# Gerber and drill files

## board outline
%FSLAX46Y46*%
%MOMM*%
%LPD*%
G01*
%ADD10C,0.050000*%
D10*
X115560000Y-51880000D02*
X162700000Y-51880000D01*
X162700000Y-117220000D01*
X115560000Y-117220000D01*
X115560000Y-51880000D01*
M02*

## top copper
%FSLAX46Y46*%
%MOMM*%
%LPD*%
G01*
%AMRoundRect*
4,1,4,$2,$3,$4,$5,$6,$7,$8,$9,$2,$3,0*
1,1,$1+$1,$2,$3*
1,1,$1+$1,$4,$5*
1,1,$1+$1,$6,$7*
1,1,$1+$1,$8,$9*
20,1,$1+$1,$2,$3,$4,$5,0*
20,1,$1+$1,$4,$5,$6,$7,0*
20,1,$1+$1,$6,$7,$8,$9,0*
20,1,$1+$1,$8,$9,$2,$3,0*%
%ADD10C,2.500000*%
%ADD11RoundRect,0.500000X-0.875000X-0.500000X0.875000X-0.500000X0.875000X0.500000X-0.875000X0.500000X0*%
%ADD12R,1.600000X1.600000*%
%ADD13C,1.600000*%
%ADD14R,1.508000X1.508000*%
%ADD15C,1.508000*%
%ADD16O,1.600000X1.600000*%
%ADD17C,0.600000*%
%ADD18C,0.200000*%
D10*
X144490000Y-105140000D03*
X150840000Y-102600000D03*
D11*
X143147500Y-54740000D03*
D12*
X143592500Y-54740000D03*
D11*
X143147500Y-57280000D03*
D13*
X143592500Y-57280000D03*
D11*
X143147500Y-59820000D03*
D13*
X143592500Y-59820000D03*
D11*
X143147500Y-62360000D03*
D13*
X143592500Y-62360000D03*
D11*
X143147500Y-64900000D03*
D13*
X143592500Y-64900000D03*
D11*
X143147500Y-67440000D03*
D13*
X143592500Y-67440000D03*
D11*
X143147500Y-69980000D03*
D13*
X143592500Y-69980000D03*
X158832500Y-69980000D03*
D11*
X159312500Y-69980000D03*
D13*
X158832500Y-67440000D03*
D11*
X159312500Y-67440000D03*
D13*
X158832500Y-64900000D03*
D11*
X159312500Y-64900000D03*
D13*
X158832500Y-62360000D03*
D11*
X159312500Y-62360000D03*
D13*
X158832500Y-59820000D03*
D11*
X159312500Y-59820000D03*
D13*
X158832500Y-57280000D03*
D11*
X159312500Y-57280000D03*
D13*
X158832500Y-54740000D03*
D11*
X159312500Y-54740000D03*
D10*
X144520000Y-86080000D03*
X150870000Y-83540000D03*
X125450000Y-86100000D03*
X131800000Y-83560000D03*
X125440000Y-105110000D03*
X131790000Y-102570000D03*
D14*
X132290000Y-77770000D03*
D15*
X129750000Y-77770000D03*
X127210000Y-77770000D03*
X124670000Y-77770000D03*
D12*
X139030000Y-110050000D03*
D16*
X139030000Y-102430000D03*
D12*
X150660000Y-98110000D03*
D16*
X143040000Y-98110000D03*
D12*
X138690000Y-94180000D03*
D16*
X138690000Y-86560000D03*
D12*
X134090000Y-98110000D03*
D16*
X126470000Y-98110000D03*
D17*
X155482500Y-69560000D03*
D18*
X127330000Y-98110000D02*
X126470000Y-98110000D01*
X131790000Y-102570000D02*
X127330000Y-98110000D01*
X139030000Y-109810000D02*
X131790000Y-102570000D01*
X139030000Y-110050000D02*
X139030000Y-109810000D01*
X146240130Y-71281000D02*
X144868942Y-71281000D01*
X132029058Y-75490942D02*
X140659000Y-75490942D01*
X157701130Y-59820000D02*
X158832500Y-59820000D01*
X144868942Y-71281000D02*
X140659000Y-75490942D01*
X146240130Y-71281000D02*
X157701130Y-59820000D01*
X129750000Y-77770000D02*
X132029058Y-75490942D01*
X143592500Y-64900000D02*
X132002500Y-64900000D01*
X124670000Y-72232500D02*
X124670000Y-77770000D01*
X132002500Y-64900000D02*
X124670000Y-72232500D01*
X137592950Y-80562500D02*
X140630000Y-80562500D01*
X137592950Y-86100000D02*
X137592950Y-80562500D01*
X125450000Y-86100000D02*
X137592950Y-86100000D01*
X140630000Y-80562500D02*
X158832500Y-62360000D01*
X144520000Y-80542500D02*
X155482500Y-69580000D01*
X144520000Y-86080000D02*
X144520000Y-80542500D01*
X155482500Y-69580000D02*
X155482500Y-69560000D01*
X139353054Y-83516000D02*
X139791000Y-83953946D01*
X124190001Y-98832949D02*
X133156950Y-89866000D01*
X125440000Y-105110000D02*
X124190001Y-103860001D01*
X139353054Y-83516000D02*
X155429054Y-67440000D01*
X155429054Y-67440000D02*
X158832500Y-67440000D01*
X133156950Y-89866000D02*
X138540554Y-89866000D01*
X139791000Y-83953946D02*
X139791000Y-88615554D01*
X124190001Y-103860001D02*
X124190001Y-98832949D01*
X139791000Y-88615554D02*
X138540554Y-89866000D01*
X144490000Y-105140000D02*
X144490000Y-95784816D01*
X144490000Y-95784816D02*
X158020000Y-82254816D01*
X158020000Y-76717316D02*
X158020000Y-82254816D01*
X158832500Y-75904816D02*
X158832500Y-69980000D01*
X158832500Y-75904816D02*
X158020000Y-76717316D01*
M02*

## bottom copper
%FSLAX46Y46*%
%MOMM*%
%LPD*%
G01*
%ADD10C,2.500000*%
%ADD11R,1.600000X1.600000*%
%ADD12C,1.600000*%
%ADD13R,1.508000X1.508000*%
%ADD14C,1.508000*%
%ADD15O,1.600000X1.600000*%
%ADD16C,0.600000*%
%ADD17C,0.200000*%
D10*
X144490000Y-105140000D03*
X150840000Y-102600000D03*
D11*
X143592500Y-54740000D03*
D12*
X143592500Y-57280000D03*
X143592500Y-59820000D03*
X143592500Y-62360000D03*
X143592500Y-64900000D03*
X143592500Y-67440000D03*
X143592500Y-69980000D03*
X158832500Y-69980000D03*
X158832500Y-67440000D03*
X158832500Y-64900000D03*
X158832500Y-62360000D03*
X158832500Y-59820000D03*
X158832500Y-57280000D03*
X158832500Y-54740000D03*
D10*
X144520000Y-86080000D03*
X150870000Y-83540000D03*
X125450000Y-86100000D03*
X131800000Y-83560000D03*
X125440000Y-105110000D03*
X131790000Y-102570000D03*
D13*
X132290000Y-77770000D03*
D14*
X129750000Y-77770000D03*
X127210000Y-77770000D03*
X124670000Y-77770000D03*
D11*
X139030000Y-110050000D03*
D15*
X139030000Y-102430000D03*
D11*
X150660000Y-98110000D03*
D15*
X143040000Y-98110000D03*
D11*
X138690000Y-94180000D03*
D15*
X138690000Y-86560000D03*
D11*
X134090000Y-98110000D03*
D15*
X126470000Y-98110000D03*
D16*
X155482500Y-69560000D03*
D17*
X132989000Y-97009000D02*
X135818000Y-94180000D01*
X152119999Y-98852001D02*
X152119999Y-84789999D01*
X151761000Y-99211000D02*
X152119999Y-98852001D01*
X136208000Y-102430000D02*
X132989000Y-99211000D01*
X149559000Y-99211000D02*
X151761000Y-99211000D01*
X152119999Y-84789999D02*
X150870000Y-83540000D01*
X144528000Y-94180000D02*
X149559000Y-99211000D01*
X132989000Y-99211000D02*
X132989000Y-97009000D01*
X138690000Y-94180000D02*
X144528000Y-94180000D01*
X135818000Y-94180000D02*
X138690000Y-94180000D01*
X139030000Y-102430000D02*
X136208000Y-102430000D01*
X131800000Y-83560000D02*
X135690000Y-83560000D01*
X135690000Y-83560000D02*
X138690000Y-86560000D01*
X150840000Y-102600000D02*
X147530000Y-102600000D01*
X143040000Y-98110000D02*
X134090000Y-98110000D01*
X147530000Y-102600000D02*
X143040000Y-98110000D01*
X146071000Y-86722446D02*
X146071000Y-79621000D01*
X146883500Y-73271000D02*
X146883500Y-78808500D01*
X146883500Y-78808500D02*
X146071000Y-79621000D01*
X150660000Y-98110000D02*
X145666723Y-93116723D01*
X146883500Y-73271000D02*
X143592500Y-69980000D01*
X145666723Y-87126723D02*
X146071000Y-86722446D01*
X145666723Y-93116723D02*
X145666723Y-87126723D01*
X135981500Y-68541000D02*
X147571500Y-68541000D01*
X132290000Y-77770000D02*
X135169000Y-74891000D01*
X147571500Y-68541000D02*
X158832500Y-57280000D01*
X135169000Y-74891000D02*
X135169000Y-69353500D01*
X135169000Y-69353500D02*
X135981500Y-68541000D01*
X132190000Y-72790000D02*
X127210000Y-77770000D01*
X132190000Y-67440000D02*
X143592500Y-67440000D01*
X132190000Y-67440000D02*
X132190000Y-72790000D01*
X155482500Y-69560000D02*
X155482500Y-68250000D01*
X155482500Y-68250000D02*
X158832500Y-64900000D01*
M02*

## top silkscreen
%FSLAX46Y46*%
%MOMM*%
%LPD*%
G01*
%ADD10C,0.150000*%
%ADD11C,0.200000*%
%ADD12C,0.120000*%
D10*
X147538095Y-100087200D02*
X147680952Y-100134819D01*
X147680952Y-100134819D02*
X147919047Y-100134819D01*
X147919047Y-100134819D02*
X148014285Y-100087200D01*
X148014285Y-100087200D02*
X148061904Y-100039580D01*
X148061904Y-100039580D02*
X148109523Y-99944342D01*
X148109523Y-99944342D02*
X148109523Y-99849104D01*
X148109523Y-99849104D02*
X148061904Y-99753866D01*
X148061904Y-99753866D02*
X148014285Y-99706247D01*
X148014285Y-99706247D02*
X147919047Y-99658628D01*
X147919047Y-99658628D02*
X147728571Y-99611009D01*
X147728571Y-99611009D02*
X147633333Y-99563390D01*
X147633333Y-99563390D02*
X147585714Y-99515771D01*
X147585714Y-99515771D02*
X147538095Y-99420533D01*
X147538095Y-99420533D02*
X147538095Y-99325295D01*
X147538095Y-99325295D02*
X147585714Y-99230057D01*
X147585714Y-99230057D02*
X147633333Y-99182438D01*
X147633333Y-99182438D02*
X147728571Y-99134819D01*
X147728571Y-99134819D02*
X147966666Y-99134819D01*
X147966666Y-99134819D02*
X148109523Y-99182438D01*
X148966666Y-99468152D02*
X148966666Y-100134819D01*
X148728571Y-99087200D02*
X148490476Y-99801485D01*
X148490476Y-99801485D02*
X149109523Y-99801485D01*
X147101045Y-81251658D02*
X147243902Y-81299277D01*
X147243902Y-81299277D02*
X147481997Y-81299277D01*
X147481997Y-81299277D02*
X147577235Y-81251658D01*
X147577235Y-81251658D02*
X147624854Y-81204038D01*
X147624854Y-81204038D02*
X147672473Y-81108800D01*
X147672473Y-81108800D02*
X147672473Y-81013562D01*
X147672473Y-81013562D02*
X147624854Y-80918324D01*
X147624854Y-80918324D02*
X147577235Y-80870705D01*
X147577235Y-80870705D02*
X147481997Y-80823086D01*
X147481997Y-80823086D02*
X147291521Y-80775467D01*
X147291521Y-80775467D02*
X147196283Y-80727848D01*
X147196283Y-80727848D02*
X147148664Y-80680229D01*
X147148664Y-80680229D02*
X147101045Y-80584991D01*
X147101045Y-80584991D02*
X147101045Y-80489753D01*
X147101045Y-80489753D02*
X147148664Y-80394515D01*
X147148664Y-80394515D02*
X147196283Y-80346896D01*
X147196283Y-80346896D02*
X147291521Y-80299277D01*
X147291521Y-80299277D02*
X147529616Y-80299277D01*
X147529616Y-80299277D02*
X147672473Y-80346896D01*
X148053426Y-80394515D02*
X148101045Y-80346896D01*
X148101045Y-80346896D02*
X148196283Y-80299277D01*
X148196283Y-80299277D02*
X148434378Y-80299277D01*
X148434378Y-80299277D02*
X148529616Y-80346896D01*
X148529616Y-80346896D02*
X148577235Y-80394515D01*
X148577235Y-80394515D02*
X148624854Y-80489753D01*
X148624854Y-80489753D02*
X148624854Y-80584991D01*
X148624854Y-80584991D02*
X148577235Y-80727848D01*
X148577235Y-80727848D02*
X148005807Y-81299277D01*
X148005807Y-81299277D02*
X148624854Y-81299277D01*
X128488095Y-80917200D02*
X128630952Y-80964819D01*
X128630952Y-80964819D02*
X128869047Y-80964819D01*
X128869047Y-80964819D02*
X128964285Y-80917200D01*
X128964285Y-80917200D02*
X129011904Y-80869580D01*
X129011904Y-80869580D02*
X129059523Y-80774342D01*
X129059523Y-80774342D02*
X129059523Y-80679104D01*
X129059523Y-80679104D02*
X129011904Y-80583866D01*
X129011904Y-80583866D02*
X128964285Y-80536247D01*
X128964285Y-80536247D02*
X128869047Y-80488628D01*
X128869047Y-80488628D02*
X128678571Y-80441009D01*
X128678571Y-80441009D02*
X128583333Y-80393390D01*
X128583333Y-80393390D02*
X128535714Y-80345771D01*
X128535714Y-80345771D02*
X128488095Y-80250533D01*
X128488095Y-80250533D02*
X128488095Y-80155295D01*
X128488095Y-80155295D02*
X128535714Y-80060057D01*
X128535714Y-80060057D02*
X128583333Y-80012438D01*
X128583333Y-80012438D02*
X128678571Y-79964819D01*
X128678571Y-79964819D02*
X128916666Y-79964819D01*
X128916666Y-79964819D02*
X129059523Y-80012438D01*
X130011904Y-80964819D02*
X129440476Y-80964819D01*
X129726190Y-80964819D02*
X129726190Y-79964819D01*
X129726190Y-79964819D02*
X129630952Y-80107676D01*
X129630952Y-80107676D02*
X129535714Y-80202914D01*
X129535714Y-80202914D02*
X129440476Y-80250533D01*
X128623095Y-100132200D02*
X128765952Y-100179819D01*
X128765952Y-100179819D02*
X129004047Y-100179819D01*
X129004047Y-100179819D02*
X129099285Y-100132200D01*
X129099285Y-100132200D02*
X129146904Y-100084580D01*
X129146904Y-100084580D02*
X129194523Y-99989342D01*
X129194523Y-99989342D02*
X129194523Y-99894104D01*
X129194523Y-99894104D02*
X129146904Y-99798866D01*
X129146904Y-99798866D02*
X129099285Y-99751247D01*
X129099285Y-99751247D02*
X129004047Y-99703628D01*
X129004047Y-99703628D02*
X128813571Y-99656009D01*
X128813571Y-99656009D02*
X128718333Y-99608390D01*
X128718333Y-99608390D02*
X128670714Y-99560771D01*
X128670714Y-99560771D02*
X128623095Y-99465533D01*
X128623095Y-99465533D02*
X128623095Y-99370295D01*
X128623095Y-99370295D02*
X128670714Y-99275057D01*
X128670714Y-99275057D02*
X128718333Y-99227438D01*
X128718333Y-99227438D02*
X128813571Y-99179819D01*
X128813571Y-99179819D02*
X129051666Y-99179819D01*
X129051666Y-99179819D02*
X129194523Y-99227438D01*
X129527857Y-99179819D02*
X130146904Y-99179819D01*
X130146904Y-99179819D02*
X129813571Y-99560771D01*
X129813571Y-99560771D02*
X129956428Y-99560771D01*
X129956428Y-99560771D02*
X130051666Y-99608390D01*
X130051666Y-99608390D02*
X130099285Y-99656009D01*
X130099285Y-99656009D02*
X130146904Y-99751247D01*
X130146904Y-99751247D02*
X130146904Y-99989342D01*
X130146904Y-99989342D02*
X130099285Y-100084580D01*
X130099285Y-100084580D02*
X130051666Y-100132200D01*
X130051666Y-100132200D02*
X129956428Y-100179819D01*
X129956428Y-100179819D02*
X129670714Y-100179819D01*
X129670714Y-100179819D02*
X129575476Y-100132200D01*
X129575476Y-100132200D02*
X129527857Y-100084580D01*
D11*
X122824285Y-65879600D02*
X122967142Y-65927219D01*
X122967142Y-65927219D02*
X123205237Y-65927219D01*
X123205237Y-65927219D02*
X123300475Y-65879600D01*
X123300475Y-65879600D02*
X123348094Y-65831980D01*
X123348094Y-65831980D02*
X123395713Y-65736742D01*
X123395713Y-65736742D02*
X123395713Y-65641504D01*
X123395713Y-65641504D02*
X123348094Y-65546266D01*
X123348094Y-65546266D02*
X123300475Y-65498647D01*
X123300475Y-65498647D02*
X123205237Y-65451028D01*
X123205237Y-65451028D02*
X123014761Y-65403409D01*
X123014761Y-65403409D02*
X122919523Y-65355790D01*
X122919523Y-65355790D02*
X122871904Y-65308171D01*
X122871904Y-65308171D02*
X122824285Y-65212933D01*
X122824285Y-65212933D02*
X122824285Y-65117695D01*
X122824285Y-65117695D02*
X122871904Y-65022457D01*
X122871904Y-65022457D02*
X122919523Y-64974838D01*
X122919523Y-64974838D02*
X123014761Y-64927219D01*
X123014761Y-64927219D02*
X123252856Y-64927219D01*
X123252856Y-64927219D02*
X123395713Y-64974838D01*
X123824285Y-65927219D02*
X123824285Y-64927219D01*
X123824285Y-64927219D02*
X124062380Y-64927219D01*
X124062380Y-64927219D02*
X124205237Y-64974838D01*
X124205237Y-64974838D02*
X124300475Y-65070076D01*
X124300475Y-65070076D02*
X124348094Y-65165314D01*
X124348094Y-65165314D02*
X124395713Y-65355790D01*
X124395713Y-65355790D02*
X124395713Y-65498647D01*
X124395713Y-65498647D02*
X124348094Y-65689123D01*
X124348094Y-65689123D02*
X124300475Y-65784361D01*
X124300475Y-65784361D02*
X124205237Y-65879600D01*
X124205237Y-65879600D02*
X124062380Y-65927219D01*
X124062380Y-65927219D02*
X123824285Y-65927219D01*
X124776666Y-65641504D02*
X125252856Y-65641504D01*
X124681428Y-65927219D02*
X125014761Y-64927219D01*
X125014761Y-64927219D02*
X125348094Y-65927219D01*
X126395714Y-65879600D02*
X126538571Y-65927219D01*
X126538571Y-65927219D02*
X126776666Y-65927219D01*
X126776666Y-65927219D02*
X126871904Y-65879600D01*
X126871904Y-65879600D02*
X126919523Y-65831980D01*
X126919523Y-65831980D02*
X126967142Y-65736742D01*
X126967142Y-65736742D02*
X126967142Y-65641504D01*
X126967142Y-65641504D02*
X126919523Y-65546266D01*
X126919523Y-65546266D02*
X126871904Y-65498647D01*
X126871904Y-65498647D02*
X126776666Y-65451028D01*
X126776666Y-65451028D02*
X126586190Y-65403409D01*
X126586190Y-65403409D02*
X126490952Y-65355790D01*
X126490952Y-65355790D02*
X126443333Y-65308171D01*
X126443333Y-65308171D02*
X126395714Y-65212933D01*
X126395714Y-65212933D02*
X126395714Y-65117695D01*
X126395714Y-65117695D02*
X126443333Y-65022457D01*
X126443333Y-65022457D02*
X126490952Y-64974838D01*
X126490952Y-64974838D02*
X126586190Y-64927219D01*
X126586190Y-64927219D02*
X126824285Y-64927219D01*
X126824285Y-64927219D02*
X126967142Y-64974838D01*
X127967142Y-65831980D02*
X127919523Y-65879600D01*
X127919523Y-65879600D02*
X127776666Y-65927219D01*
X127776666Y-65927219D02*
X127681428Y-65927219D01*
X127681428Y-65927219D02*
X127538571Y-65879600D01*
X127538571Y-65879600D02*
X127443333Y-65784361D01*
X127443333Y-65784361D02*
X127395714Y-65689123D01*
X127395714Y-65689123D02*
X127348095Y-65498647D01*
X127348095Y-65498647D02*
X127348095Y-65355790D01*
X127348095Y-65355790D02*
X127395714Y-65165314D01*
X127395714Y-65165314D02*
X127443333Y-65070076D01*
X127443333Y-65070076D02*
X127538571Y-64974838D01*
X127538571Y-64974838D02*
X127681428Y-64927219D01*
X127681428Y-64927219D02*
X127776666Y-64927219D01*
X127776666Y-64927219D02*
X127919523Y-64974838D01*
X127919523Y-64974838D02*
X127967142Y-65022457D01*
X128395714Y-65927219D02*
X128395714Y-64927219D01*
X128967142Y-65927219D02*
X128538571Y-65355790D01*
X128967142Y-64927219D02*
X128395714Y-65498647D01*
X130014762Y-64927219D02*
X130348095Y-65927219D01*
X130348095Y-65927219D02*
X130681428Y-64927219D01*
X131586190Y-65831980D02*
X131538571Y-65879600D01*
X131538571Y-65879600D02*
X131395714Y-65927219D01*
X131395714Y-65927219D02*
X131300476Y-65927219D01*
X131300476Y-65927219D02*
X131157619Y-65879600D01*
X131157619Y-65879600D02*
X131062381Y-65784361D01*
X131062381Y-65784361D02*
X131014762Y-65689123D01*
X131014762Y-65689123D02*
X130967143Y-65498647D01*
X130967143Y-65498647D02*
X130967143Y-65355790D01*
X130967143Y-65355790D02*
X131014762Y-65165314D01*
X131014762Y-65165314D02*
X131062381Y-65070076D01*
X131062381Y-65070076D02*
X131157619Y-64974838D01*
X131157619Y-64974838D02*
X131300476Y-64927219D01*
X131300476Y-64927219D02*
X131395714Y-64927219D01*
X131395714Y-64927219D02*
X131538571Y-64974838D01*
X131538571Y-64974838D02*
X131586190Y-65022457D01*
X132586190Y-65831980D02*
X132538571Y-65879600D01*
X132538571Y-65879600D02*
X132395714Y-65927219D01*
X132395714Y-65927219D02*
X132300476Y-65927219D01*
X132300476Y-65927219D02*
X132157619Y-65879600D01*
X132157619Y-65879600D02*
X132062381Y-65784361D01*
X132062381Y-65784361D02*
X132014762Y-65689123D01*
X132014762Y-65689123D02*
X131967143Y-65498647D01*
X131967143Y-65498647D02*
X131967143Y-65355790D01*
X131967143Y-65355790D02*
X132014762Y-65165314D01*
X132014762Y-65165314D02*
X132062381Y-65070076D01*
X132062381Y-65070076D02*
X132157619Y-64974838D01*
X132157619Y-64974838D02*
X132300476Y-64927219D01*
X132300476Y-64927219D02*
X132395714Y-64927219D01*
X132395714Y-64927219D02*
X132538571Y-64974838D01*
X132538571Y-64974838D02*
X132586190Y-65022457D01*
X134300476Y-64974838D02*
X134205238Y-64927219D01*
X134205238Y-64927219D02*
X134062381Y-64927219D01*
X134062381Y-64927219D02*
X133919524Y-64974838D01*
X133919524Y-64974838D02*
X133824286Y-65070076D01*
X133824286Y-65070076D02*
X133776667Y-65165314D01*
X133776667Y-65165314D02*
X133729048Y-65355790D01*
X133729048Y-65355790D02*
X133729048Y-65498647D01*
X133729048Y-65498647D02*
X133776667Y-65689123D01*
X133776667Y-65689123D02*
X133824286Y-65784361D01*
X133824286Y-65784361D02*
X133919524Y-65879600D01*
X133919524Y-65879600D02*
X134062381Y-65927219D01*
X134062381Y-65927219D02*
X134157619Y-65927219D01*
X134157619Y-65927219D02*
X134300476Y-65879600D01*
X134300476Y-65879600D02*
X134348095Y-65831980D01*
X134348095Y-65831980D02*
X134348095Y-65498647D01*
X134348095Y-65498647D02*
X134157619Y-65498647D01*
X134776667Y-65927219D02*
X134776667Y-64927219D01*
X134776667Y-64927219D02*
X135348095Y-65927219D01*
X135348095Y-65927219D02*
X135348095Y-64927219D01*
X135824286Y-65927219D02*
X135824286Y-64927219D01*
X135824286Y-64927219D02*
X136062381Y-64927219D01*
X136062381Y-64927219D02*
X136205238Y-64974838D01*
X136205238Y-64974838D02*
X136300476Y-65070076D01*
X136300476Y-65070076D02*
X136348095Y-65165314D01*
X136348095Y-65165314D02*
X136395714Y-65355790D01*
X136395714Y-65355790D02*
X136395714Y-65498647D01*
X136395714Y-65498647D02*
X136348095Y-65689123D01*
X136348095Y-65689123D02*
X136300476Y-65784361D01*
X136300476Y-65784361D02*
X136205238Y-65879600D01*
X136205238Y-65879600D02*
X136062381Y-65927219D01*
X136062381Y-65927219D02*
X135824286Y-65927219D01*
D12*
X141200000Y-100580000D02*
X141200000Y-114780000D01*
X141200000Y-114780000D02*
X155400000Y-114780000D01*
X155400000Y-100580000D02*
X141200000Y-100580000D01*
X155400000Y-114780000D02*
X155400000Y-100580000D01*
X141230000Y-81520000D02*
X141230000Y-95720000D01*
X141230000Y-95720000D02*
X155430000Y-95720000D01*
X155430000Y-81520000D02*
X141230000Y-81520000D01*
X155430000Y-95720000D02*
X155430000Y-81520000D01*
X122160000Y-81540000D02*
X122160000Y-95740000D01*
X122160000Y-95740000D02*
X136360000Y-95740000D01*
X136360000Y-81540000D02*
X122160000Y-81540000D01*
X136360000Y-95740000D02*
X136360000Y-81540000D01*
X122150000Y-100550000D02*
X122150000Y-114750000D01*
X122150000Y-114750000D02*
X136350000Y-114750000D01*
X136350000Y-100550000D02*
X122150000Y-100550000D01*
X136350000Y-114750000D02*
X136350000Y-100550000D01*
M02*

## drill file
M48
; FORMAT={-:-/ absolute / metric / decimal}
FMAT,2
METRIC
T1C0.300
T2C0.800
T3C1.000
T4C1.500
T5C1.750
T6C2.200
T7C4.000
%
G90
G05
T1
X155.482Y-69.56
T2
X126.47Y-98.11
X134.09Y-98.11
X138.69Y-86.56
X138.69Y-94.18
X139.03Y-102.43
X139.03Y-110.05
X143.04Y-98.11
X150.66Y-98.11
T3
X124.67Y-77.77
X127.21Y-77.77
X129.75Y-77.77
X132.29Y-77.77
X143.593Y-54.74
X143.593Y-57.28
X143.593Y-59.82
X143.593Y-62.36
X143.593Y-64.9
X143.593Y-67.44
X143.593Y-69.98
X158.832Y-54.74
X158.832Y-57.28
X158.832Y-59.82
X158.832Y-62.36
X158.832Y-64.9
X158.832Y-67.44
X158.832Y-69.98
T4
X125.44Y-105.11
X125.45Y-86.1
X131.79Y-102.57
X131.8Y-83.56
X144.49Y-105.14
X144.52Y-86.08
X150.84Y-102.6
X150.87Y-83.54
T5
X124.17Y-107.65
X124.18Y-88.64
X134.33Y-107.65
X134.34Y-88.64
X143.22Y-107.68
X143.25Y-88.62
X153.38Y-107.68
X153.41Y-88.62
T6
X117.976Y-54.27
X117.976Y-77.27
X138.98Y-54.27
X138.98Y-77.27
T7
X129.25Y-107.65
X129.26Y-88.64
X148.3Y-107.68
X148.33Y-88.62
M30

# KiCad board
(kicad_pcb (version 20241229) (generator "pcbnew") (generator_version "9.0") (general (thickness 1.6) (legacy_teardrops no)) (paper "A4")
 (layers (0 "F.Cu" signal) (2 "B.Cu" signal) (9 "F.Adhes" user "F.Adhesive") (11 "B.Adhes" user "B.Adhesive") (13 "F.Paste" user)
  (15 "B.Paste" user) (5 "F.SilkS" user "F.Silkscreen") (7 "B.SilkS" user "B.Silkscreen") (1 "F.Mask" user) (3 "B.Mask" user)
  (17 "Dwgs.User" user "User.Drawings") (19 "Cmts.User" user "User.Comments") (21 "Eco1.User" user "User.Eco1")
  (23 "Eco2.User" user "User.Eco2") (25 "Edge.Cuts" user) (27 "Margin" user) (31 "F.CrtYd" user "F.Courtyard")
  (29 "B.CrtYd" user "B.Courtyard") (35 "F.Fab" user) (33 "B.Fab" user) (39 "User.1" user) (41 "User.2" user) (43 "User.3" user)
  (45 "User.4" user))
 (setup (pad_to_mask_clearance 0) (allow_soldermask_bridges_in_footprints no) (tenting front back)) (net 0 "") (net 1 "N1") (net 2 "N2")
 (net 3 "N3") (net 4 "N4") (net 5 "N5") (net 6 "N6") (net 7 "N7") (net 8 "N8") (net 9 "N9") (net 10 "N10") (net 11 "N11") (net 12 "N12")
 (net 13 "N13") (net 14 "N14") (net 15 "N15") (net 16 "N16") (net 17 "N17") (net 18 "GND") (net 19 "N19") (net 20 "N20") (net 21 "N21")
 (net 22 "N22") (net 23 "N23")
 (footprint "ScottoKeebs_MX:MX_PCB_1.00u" (layer "F.Cu") (at 148.3 107.68)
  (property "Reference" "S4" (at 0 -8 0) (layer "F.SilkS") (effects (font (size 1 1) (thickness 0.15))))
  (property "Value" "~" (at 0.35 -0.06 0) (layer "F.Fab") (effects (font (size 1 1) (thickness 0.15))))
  (fp_line (start -7.1 -7.1) (end -7.1 7.1) (stroke (width 0.12) (type solid)) (layer "F.SilkS"))
  (fp_line (start -7.1 7.1) (end 7.1 7.1) (stroke (width 0.12) (type solid)) (layer "F.SilkS"))
  (fp_line (start 7.1 -7.1) (end -7.1 -7.1) (stroke (width 0.12) (type solid)) (layer "F.SilkS"))
  (fp_line (start 7.1 7.1) (end 7.1 -7.1) (stroke (width 0.12) (type solid)) (layer "F.SilkS"))
  (pad "" np_thru_hole circle (at -5.08 0) (size 1.75 1.75) (drill 1.75) (layers "*.Cu" "*.Mask"))
  (pad "" np_thru_hole circle (at 0 0) (size 4 4) (drill 4) (layers "*.Cu" "*.Mask"))
  (pad "" np_thru_hole circle (at 5.08 0) (size 1.75 1.75) (drill 1.75) (layers "*.Cu" "*.Mask"))
  (pad "1" thru_hole circle (at -3.81 -2.54) (size 2.5 2.5) (drill 1.5) (layers "*.Cu" "*.Mask") (remove_unused_layers no) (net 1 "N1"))
  (pad "2" thru_hole circle (at 2.54 -5.08) (size 2.5 2.5) (drill 1.5) (layers "*.Cu" "*.Mask") (remove_unused_layers no) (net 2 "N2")))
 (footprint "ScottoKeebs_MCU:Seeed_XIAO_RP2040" (layer "F.Cu") (at 151.2125 62.36)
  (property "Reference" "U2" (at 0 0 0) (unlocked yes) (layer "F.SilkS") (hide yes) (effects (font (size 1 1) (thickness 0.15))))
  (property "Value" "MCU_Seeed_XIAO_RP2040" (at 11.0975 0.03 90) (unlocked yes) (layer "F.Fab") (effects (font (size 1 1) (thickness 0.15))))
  (pad "1" smd roundrect (at -8.065 -7.62) (size 2.75 2) (layers "F.Cu" "F.Mask" "F.Paste") (roundrect_rratio 0.25) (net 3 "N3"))
  (pad "1" thru_hole rect (at -7.62 -7.62 90) (size 1.6 1.6) (drill 1) (layers "*.Cu" "*.Mask") (remove_unused_layers no) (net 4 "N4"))
  (pad "2" smd roundrect (at -8.065 -5.08) (size 2.75 2) (layers "F.Cu" "F.Mask" "F.Paste") (roundrect_rratio 0.25) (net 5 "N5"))
  (pad "2" thru_hole circle (at -7.62 -5.08 90) (size 1.6 1.6) (drill 1) (layers "*.Cu" "*.Mask") (remove_unused_layers no) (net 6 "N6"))
  (pad "3" smd roundrect (at -8.065 -2.54) (size 2.75 2) (layers "F.Cu" "F.Mask" "F.Paste") (roundrect_rratio 0.25) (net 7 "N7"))
  (pad "3" thru_hole circle (at -7.62 -2.54 90) (size 1.6 1.6) (drill 1) (layers "*.Cu" "*.Mask") (remove_unused_layers no) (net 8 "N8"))
  (pad "4" smd roundrect (at -8.065 0) (size 2.75 2) (layers "F.Cu" "F.Mask" "F.Paste") (roundrect_rratio 0.25) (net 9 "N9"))
  (pad "4" thru_hole circle (at -7.62 0 90) (size 1.6 1.6) (drill 1) (layers "*.Cu" "*.Mask") (remove_unused_layers no) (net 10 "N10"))
  (pad "5" smd roundrect (at -8.065 2.54) (size 2.75 2) (layers "F.Cu" "F.Mask" "F.Paste") (roundrect_rratio 0.25) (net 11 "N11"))
  (pad "5" thru_hole circle (at -7.62 2.54 90) (size 1.6 1.6) (drill 1) (layers "*.Cu" "*.Mask") (remove_unused_layers no) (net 11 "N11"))
  (pad "6" smd roundrect (at -8.065 5.08) (size 2.75 2) (layers "F.Cu" "F.Mask" "F.Paste") (roundrect_rratio 0.25) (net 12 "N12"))
  (pad "6" thru_hole circle (at -7.62 5.08 90) (size 1.6 1.6) (drill 1) (layers "*.Cu" "*.Mask") (remove_unused_layers no) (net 12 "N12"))
  (pad "7" smd roundrect (at -8.065 7.62) (size 2.75 2) (layers "F.Cu" "F.Mask" "F.Paste") (roundrect_rratio 0.25) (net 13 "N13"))
  (pad "7" thru_hole circle (at -7.62 7.62 90) (size 1.6 1.6) (drill 1) (layers "*.Cu" "*.Mask") (remove_unused_layers no) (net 13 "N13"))
  (pad "8" thru_hole circle (at 7.62 7.62 90) (size 1.6 1.6) (drill 1) (layers "*.Cu" "*.Mask") (remove_unused_layers no) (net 1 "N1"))
  (pad "8" smd roundrect (at 8.1 7.62) (size 2.75 2) (layers "F.Cu" "F.Mask" "F.Paste") (roundrect_rratio 0.25) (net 1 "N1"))
  (pad "9" thru_hole circle (at 7.62 5.08 90) (size 1.6 1.6) (drill 1) (layers "*.Cu" "*.Mask") (remove_unused_layers no) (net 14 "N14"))
  (pad "9" smd roundrect (at 8.1 5.08) (size 2.75 2) (layers "F.Cu" "F.Mask" "F.Paste") (roundrect_rratio 0.25) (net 14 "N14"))
  (pad "10" thru_hole circle (at 7.62 2.54 90) (size 1.6 1.6) (drill 1) (layers "*.Cu" "*.Mask") (remove_unused_layers no) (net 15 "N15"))
  (pad "10" smd roundrect (at 8.1 2.54) (size 2.75 2) (layers "F.Cu" "F.Mask" "F.Paste") (roundrect_rratio 0.25) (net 15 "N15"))
  (pad "11" thru_hole circle (at 7.62 0 90) (size 1.6 1.6) (drill 1) (layers "*.Cu" "*.Mask") (remove_unused_layers no) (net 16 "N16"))
  (pad "11" smd roundrect (at 8.1 0) (size 2.75 2) (layers "F.Cu" "F.Mask" "F.Paste") (roundrect_rratio 0.25) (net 16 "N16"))
  (pad "12" thru_hole circle (at 7.62 -2.54 90) (size 1.6 1.6) (drill 1) (layers "*.Cu" "*.Mask") (remove_unused_layers no) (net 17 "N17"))
  (pad "12" smd roundrect (at 8.1 -2.54) (size 2.75 2) (layers "F.Cu" "F.Mask" "F.Paste") (roundrect_rratio 0.25) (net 17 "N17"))
  (pad "13" thru_hole circle (at 7.62 -5.08 90) (size 1.6 1.6) (drill 1) (layers "*.Cu" "*.Mask") (remove_unused_layers no) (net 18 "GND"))
  (pad "13" smd roundrect (at 8.1 -5.08) (size 2.75 2) (layers "F.Cu" "F.Mask" "F.Paste") (roundrect_rratio 0.25) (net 18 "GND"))
  (pad "14" thru_hole circle (at 7.62 -7.62 90) (size 1.6 1.6) (drill 1) (layers "*.Cu" "*.Mask") (remove_unused_layers no) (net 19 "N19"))
  (pad "14" smd roundrect (at 8.1 -7.62) (size 2.75 2) (layers "F.Cu" "F.Mask" "F.Paste") (roundrect_rratio 0.25) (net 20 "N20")))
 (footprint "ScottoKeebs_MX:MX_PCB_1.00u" (layer "F.Cu") (at 148.33 88.62)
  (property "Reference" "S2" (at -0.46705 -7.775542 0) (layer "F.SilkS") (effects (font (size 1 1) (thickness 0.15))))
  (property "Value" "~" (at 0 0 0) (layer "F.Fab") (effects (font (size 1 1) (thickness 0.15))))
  (fp_line (start -7.1 -7.1) (end -7.1 7.1) (stroke (width 0.12) (type solid)) (layer "F.SilkS"))
  (fp_line (start -7.1 7.1) (end 7.1 7.1) (stroke (width 0.12) (type solid)) (layer "F.SilkS"))
  (fp_line (start 7.1 -7.1) (end -7.1 -7.1) (stroke (width 0.12) (type solid)) (layer "F.SilkS"))
  (fp_line (start 7.1 7.1) (end 7.1 -7.1) (stroke (width 0.12) (type solid)) (layer "F.SilkS"))
  (pad "" np_thru_hole circle (at -5.08 0) (size 1.75 1.75) (drill 1.75) (layers "*.Cu" "*.Mask"))
  (pad "" np_thru_hole circle (at 0 0) (size 4 4) (drill 4) (layers "*.Cu" "*.Mask"))
  (pad "" np_thru_hole circle (at 5.08 0) (size 1.75 1.75) (drill 1.75) (layers "*.Cu" "*.Mask"))
  (pad "1" thru_hole circle (at -3.81 -2.54) (size 2.5 2.5) (drill 1.5) (layers "*.Cu" "*.Mask") (remove_unused_layers no) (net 15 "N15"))
  (pad "2" thru_hole circle (at 2.54 -5.08) (size 2.5 2.5) (drill 1.5) (layers "*.Cu" "*.Mask") (remove_unused_layers no) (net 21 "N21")))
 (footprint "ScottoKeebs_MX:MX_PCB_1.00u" (layer "F.Cu") (at 129.26 88.64)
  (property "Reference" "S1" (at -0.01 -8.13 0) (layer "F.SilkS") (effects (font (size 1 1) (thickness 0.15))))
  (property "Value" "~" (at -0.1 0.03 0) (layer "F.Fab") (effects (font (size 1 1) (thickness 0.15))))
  (fp_line (start -7.1 -7.1) (end -7.1 7.1) (stroke (width 0.12) (type solid)) (layer "F.SilkS"))
  (fp_line (start -7.1 7.1) (end 7.1 7.1) (stroke (width 0.12) (type solid)) (layer "F.SilkS"))
  (fp_line (start 7.1 -7.1) (end -7.1 -7.1) (stroke (width 0.12) (type solid)) (layer "F.SilkS"))
  (fp_line (start 7.1 7.1) (end 7.1 -7.1) (stroke (width 0.12) (type solid)) (layer "F.SilkS"))
  (pad "" np_thru_hole circle (at -5.08 0) (size 1.75 1.75) (drill 1.75) (layers "*.Cu" "*.Mask"))
  (pad "" np_thru_hole circle (at 0 0) (size 4 4) (drill 4) (layers "*.Cu" "*.Mask"))
  (pad "" np_thru_hole circle (at 5.08 0) (size 1.75 1.75) (drill 1.75) (layers "*.Cu" "*.Mask"))
  (pad "1" thru_hole circle (at -3.81 -2.54) (size 2.5 2.5) (drill 1.5) (layers "*.Cu" "*.Mask") (remove_unused_layers no) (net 16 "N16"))
  (pad "2" thru_hole circle (at 2.54 -5.08) (size 2.5 2.5) (drill 1.5) (layers "*.Cu" "*.Mask") (remove_unused_layers no) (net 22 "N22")))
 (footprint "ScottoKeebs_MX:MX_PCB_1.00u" (layer "F.Cu") (at 129.25 107.65)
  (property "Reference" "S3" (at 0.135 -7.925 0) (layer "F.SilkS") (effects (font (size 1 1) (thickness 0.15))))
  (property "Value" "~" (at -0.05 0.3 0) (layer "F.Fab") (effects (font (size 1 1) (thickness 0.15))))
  (fp_line (start -7.1 -7.1) (end -7.1 7.1) (stroke (width 0.12) (type solid)) (layer "F.SilkS"))
  (fp_line (start -7.1 7.1) (end 7.1 7.1) (stroke (width 0.12) (type solid)) (layer "F.SilkS"))
  (fp_line (start 7.1 -7.1) (end -7.1 -7.1) (stroke (width 0.12) (type solid)) (layer "F.SilkS"))
  (fp_line (start 7.1 7.1) (end 7.1 -7.1) (stroke (width 0.12) (type solid)) (layer "F.SilkS"))
  (pad "" np_thru_hole circle (at -5.08 0) (size 1.75 1.75) (drill 1.75) (layers "*.Cu" "*.Mask"))
  (pad "" np_thru_hole circle (at 0 0) (size 4 4) (drill 4) (layers "*.Cu" "*.Mask"))
  (pad "" np_thru_hole circle (at 5.08 0) (size 1.75 1.75) (drill 1.75) (layers "*.Cu" "*.Mask"))
  (pad "1" thru_hole circle (at -3.81 -2.54) (size 2.5 2.5) (drill 1.5) (layers "*.Cu" "*.Mask") (remove_unused_layers no) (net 14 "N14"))
  (pad "2" thru_hole circle (at 2.54 -5.08) (size 2.5 2.5) (drill 1.5) (layers "*.Cu" "*.Mask") (remove_unused_layers no) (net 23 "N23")))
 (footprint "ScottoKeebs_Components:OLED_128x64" (layer "F.Cu") (at 128.48 65.77)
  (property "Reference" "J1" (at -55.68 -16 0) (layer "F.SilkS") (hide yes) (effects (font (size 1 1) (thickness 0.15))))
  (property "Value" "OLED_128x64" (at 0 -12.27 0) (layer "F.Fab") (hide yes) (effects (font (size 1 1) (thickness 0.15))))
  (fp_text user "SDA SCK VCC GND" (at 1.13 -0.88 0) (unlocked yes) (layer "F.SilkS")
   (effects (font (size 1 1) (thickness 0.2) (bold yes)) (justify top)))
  (pad "" np_thru_hole circle (at -10.50445 -11.5 180) (size 2.2 2.2) (drill 2.2) (layers "*.Cu" "*.Mask") (solder_mask_margin 0.102))
  (pad "" np_thru_hole circle (at -10.50445 11.5 180) (size 2.2 2.2) (drill 2.2) (layers "*.Cu" "*.Mask") (solder_mask_margin 0.102))
  (pad "" np_thru_hole circle (at 10.5 -11.5 180) (size 2.2 2.2) (drill 2.2) (layers "*.Cu" "*.Mask") (solder_mask_margin 0.102))
  (pad "" np_thru_hole circle (at 10.5 11.5 180) (size 2.2 2.2) (drill 2.2) (layers "*.Cu" "*.Mask") (solder_mask_margin 0.102))
  (pad "1" thru_hole rect (at 3.81 12 180) (size 1.508 1.508) (drill 1) (layers "*.Cu" "*.Mask") (remove_unused_layers no) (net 18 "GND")
   (solder_mask_margin 0.102))
  (pad "2" thru_hole circle (at 1.27 12 180) (size 1.508 1.508) (drill 1) (layers "*.Cu" "*.Mask") (remove_unused_layers no) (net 17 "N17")
   (solder_mask_margin 0.102))
  (pad "3" thru_hole circle (at -1.27 12 180) (size 1.508 1.508) (drill 1) (layers "*.Cu" "*.Mask") (remove_unused_layers no) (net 12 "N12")
   (solder_mask_margin 0.102))
  (pad "4" thru_hole circle (at -3.81 12 180) (size 1.508 1.508) (drill 1) (layers "*.Cu" "*.Mask") (remove_unused_layers no) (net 11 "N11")
   (solder_mask_margin 0.102)))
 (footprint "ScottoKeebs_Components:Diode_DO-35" (layer "B.Cu") (at 139.03 110.05 90)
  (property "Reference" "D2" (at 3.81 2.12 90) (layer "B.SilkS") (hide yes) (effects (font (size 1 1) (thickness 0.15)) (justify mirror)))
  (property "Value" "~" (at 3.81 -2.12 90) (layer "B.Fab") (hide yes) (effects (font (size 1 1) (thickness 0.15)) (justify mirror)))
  (pad "1" thru_hole rect (at 0 0 90) (size 1.6 1.6) (drill 0.8) (layers "*.Cu" "*.Mask") (remove_unused_layers no) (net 23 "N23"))
  (pad "2" thru_hole oval (at 7.62 0 90) (size 1.6 1.6) (drill 0.8) (layers "*.Cu" "*.Mask") (remove_unused_layers no) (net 21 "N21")))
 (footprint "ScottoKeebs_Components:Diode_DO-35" (layer "B.Cu") (at 150.66 98.11 180)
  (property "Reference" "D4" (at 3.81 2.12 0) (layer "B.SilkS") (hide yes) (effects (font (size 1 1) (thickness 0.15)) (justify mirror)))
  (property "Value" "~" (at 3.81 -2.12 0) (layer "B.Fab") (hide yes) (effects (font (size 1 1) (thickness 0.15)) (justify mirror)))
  (pad "1" thru_hole rect (at 0 0 180) (size 1.6 1.6) (drill 0.8) (layers "*.Cu" "*.Mask") (remove_unused_layers no) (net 13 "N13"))
  (pad "2" thru_hole oval (at 7.62 0 180) (size 1.6 1.6) (drill 0.8) (layers "*.Cu" "*.Mask") (remove_unused_layers no) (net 2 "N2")))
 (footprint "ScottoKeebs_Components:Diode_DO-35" (layer "B.Cu") (at 138.69 94.18 90)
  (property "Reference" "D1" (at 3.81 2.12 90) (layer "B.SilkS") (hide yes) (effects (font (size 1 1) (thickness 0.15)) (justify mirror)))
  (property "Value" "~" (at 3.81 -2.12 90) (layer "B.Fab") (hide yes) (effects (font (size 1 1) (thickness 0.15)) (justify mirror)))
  (pad "1" thru_hole rect (at 0 0 90) (size 1.6 1.6) (drill 0.8) (layers "*.Cu" "*.Mask") (remove_unused_layers no) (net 21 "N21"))
  (pad "2" thru_hole oval (at 7.62 0 90) (size 1.6 1.6) (drill 0.8) (layers "*.Cu" "*.Mask") (remove_unused_layers no) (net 22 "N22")))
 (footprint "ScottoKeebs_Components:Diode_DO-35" (layer "B.Cu") (at 134.09 98.11 180)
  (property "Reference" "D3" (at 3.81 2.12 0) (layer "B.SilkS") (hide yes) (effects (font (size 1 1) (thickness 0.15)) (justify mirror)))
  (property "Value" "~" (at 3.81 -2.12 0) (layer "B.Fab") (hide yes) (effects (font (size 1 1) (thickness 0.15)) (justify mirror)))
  (pad "1" thru_hole rect (at 0 0 180) (size 1.6 1.6) (drill 0.8) (layers "*.Cu" "*.Mask") (remove_unused_layers no) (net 2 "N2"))
  (pad "2" thru_hole oval (at 7.62 0 180) (size 1.6 1.6) (drill 0.8) (layers "*.Cu" "*.Mask") (remove_unused_layers no) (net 23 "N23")))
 (gr_rect (start 115.56 51.88) (end 162.7 117.22) (stroke (width 0.05) (type default)) (fill no) (layer "Edge.Cuts"))
 (segment (start 132.989 97.009) (end 135.818 94.18) (width 0.2) (layer "B.Cu") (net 21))
 (segment (start 152.119999 98.852001) (end 152.119999 84.789999) (width 0.2) (layer "B.Cu") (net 21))
 (segment (start 151.761 99.211) (end 152.119999 98.852001) (width 0.2) (layer "B.Cu") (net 21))
 (segment (start 136.208 102.43) (end 132.989 99.211) (width 0.2) (layer "B.Cu") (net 21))
 (segment (start 149.559 99.211) (end 151.761 99.211) (width 0.2) (layer "B.Cu") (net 21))
 (segment (start 152.119999 84.789999) (end 150.87 83.54) (width 0.2) (layer "B.Cu") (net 21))
 (segment (start 144.528 94.18) (end 149.559 99.211) (width 0.2) (layer "B.Cu") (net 21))
 (segment (start 132.989 99.211) (end 132.989 97.009) (width 0.2) (layer "B.Cu") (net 21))
 (segment (start 138.69 94.18) (end 144.528 94.18) (width 0.2) (layer "B.Cu") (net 21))
 (segment (start 135.818 94.18) (end 138.69 94.18) (width 0.2) (layer "B.Cu") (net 21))
 (segment (start 139.03 102.43) (end 136.208 102.43) (width 0.2) (layer "B.Cu") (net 21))
 (segment (start 131.8 83.56) (end 135.69 83.56) (width 0.2) (layer "B.Cu") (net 22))
 (segment (start 135.69 83.56) (end 138.69 86.56) (width 0.2) (layer "B.Cu") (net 22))
 (segment (start 127.33 98.11) (end 126.47 98.11) (width 0.2) (layer "F.Cu") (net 23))
 (segment (start 131.79 102.57) (end 127.33 98.11) (width 0.2) (layer "F.Cu") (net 23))
 (segment (start 139.03 109.81) (end 131.79 102.57) (width 0.2) (layer "F.Cu") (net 23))
 (segment (start 139.03 110.05) (end 139.03 109.81) (width 0.2) (layer "F.Cu") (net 23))
 (segment (start 150.84 102.6) (end 147.53 102.6) (width 0.2) (layer "B.Cu") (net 2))
 (segment (start 143.04 98.11) (end 134.09 98.11) (width 0.2) (layer "B.Cu") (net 2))
 (segment (start 147.53 102.6) (end 143.04 98.11) (width 0.2) (layer "B.Cu") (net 2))
 (segment (start 146.071 86.722446) (end 146.071 79.621) (width 0.2) (layer "B.Cu") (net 13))
 (segment (start 146.8835 73.271) (end 146.8835 78.8085) (width 0.2) (layer "B.Cu") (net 13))
 (segment (start 146.8835 78.8085) (end 146.071 79.621) (width 0.2) (layer "B.Cu") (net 13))
 (segment (start 150.66 98.11) (end 145.666723 93.116723) (width 0.2) (layer "B.Cu") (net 13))
 (segment (start 146.8835 73.271) (end 143.5925 69.98) (width 0.2) (layer "B.Cu") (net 13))
 (segment (start 145.666723 87.126723) (end 146.071 86.722446) (width 0.2) (layer "B.Cu") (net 13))
 (segment (start 145.666723 93.116723) (end 145.666723 87.126723) (width 0.2) (layer "B.Cu") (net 13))
 (segment (start 135.9815 68.541) (end 147.5715 68.541) (width 0.2) (layer "B.Cu") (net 18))
 (segment (start 132.29 77.77) (end 135.169 74.891) (width 0.2) (layer "B.Cu") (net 18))
 (segment (start 147.5715 68.541) (end 158.8325 57.28) (width 0.2) (layer "B.Cu") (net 18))
 (segment (start 135.169 74.891) (end 135.169 69.3535) (width 0.2) (layer "B.Cu") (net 18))
 (segment (start 135.169 69.3535) (end 135.9815 68.541) (width 0.2) (layer "B.Cu") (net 18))
 (segment (start 146.24013 71.281) (end 144.868942 71.281) (width 0.2) (layer "F.Cu") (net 17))
 (segment (start 132.029058 75.490942) (end 140.659 75.490942) (width 0.2) (layer "F.Cu") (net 17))
 (segment (start 157.70113 59.82) (end 158.8325 59.82) (width 0.2) (layer "F.Cu") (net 17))
 (segment (start 144.868942 71.281) (end 140.659 75.490942) (width 0.2) (layer "F.Cu") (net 17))
 (segment (start 146.24013 71.281) (end 157.70113 59.82) (width 0.2) (layer "F.Cu") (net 17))
 (segment (start 129.75 77.77) (end 132.029058 75.490942) (width 0.2) (layer "F.Cu") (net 17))
 (segment (start 143.5925 64.9) (end 132.0025 64.9) (width 0.2) (layer "F.Cu") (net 11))
 (segment (start 124.67 72.2325) (end 124.67 77.77) (width 0.2) (layer "F.Cu") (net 11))
 (segment (start 132.0025 64.9) (end 124.67 72.2325) (width 0.2) (layer "F.Cu") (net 11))
 (segment (start 132.19 72.79) (end 127.21 77.77) (width 0.2) (layer "B.Cu") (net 12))
 (segment (start 132.19 67.44) (end 143.5925 67.44) (width 0.2) (layer "B.Cu") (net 12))
 (segment (start 132.19 67.44) (end 132.19 72.79) (width 0.2) (layer "B.Cu") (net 12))
 (segment (start 137.59295 80.5625) (end 140.63 80.5625) (width 0.2) (layer "F.Cu") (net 16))
 (segment (start 137.59295 86.1) (end 137.59295 80.5625) (width 0.2) (layer "F.Cu") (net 16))
 (segment (start 125.45 86.1) (end 137.59295 86.1) (width 0.2) (layer "F.Cu") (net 16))
 (segment (start 140.63 80.5625) (end 158.8325 62.36) (width 0.2) (layer "F.Cu") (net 16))
 (segment (start 144.52 80.5425) (end 155.4825 69.58) (width 0.2) (layer "F.Cu") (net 15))
 (segment (start 144.52 86.08) (end 144.52 80.5425) (width 0.2) (layer "F.Cu") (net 15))
 (segment (start 155.4825 69.58) (end 155.4825 69.56) (width 0.2) (layer "F.Cu") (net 15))
 (via (at 155.4825 69.56) (size 0.6) (drill 0.3) (layers "F.Cu" "B.Cu") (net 15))
 (segment (start 155.4825 69.56) (end 155.4825 68.25) (width 0.2) (layer "B.Cu") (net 15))
 (segment (start 155.4825 68.25) (end 158.8325 64.9) (width 0.2) (layer "B.Cu") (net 15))
 (segment (start 139.353054 83.516) (end 139.791 83.953946) (width 0.2) (layer "F.Cu") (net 14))
 (segment (start 124.190001 98.832949) (end 133.15695 89.866) (width 0.2) (layer "F.Cu") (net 14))
 (segment (start 125.44 105.11) (end 124.190001 103.860001) (width 0.2) (layer "F.Cu") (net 14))
 (segment (start 139.353054 83.516) (end 155.429054 67.44) (width 0.2) (layer "F.Cu") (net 14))
 (segment (start 155.429054 67.44) (end 158.8325 67.44) (width 0.2) (layer "F.Cu") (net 14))
 (segment (start 133.15695 89.866) (end 138.540554 89.866) (width 0.2) (layer "F.Cu") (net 14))
 (segment (start 139.791 83.953946) (end 139.791 88.615554) (width 0.2) (layer "F.Cu") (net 14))
 (segment (start 124.190001 103.860001) (end 124.190001 98.832949) (width 0.2) (layer "F.Cu") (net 14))
 (segment (start 139.791 88.615554) (end 138.540554 89.866) (width 0.2) (layer "F.Cu") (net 14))
 (segment (start 144.49 105.14) (end 144.49 95.784816) (width 0.2) (layer "F.Cu") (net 1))
 (segment (start 144.49 95.784816) (end 158.02 82.254816) (width 0.2) (layer "F.Cu") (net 1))
 (segment (start 158.02 76.717316) (end 158.02 82.254816) (width 0.2) (layer "F.Cu") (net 1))
 (segment (start 158.8325 75.904816) (end 158.8325 69.98) (width 0.2) (layer "F.Cu") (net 1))
 (segment (start 158.8325 75.904816) (end 158.02 76.717316) (width 0.2) (layer "F.Cu") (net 1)))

